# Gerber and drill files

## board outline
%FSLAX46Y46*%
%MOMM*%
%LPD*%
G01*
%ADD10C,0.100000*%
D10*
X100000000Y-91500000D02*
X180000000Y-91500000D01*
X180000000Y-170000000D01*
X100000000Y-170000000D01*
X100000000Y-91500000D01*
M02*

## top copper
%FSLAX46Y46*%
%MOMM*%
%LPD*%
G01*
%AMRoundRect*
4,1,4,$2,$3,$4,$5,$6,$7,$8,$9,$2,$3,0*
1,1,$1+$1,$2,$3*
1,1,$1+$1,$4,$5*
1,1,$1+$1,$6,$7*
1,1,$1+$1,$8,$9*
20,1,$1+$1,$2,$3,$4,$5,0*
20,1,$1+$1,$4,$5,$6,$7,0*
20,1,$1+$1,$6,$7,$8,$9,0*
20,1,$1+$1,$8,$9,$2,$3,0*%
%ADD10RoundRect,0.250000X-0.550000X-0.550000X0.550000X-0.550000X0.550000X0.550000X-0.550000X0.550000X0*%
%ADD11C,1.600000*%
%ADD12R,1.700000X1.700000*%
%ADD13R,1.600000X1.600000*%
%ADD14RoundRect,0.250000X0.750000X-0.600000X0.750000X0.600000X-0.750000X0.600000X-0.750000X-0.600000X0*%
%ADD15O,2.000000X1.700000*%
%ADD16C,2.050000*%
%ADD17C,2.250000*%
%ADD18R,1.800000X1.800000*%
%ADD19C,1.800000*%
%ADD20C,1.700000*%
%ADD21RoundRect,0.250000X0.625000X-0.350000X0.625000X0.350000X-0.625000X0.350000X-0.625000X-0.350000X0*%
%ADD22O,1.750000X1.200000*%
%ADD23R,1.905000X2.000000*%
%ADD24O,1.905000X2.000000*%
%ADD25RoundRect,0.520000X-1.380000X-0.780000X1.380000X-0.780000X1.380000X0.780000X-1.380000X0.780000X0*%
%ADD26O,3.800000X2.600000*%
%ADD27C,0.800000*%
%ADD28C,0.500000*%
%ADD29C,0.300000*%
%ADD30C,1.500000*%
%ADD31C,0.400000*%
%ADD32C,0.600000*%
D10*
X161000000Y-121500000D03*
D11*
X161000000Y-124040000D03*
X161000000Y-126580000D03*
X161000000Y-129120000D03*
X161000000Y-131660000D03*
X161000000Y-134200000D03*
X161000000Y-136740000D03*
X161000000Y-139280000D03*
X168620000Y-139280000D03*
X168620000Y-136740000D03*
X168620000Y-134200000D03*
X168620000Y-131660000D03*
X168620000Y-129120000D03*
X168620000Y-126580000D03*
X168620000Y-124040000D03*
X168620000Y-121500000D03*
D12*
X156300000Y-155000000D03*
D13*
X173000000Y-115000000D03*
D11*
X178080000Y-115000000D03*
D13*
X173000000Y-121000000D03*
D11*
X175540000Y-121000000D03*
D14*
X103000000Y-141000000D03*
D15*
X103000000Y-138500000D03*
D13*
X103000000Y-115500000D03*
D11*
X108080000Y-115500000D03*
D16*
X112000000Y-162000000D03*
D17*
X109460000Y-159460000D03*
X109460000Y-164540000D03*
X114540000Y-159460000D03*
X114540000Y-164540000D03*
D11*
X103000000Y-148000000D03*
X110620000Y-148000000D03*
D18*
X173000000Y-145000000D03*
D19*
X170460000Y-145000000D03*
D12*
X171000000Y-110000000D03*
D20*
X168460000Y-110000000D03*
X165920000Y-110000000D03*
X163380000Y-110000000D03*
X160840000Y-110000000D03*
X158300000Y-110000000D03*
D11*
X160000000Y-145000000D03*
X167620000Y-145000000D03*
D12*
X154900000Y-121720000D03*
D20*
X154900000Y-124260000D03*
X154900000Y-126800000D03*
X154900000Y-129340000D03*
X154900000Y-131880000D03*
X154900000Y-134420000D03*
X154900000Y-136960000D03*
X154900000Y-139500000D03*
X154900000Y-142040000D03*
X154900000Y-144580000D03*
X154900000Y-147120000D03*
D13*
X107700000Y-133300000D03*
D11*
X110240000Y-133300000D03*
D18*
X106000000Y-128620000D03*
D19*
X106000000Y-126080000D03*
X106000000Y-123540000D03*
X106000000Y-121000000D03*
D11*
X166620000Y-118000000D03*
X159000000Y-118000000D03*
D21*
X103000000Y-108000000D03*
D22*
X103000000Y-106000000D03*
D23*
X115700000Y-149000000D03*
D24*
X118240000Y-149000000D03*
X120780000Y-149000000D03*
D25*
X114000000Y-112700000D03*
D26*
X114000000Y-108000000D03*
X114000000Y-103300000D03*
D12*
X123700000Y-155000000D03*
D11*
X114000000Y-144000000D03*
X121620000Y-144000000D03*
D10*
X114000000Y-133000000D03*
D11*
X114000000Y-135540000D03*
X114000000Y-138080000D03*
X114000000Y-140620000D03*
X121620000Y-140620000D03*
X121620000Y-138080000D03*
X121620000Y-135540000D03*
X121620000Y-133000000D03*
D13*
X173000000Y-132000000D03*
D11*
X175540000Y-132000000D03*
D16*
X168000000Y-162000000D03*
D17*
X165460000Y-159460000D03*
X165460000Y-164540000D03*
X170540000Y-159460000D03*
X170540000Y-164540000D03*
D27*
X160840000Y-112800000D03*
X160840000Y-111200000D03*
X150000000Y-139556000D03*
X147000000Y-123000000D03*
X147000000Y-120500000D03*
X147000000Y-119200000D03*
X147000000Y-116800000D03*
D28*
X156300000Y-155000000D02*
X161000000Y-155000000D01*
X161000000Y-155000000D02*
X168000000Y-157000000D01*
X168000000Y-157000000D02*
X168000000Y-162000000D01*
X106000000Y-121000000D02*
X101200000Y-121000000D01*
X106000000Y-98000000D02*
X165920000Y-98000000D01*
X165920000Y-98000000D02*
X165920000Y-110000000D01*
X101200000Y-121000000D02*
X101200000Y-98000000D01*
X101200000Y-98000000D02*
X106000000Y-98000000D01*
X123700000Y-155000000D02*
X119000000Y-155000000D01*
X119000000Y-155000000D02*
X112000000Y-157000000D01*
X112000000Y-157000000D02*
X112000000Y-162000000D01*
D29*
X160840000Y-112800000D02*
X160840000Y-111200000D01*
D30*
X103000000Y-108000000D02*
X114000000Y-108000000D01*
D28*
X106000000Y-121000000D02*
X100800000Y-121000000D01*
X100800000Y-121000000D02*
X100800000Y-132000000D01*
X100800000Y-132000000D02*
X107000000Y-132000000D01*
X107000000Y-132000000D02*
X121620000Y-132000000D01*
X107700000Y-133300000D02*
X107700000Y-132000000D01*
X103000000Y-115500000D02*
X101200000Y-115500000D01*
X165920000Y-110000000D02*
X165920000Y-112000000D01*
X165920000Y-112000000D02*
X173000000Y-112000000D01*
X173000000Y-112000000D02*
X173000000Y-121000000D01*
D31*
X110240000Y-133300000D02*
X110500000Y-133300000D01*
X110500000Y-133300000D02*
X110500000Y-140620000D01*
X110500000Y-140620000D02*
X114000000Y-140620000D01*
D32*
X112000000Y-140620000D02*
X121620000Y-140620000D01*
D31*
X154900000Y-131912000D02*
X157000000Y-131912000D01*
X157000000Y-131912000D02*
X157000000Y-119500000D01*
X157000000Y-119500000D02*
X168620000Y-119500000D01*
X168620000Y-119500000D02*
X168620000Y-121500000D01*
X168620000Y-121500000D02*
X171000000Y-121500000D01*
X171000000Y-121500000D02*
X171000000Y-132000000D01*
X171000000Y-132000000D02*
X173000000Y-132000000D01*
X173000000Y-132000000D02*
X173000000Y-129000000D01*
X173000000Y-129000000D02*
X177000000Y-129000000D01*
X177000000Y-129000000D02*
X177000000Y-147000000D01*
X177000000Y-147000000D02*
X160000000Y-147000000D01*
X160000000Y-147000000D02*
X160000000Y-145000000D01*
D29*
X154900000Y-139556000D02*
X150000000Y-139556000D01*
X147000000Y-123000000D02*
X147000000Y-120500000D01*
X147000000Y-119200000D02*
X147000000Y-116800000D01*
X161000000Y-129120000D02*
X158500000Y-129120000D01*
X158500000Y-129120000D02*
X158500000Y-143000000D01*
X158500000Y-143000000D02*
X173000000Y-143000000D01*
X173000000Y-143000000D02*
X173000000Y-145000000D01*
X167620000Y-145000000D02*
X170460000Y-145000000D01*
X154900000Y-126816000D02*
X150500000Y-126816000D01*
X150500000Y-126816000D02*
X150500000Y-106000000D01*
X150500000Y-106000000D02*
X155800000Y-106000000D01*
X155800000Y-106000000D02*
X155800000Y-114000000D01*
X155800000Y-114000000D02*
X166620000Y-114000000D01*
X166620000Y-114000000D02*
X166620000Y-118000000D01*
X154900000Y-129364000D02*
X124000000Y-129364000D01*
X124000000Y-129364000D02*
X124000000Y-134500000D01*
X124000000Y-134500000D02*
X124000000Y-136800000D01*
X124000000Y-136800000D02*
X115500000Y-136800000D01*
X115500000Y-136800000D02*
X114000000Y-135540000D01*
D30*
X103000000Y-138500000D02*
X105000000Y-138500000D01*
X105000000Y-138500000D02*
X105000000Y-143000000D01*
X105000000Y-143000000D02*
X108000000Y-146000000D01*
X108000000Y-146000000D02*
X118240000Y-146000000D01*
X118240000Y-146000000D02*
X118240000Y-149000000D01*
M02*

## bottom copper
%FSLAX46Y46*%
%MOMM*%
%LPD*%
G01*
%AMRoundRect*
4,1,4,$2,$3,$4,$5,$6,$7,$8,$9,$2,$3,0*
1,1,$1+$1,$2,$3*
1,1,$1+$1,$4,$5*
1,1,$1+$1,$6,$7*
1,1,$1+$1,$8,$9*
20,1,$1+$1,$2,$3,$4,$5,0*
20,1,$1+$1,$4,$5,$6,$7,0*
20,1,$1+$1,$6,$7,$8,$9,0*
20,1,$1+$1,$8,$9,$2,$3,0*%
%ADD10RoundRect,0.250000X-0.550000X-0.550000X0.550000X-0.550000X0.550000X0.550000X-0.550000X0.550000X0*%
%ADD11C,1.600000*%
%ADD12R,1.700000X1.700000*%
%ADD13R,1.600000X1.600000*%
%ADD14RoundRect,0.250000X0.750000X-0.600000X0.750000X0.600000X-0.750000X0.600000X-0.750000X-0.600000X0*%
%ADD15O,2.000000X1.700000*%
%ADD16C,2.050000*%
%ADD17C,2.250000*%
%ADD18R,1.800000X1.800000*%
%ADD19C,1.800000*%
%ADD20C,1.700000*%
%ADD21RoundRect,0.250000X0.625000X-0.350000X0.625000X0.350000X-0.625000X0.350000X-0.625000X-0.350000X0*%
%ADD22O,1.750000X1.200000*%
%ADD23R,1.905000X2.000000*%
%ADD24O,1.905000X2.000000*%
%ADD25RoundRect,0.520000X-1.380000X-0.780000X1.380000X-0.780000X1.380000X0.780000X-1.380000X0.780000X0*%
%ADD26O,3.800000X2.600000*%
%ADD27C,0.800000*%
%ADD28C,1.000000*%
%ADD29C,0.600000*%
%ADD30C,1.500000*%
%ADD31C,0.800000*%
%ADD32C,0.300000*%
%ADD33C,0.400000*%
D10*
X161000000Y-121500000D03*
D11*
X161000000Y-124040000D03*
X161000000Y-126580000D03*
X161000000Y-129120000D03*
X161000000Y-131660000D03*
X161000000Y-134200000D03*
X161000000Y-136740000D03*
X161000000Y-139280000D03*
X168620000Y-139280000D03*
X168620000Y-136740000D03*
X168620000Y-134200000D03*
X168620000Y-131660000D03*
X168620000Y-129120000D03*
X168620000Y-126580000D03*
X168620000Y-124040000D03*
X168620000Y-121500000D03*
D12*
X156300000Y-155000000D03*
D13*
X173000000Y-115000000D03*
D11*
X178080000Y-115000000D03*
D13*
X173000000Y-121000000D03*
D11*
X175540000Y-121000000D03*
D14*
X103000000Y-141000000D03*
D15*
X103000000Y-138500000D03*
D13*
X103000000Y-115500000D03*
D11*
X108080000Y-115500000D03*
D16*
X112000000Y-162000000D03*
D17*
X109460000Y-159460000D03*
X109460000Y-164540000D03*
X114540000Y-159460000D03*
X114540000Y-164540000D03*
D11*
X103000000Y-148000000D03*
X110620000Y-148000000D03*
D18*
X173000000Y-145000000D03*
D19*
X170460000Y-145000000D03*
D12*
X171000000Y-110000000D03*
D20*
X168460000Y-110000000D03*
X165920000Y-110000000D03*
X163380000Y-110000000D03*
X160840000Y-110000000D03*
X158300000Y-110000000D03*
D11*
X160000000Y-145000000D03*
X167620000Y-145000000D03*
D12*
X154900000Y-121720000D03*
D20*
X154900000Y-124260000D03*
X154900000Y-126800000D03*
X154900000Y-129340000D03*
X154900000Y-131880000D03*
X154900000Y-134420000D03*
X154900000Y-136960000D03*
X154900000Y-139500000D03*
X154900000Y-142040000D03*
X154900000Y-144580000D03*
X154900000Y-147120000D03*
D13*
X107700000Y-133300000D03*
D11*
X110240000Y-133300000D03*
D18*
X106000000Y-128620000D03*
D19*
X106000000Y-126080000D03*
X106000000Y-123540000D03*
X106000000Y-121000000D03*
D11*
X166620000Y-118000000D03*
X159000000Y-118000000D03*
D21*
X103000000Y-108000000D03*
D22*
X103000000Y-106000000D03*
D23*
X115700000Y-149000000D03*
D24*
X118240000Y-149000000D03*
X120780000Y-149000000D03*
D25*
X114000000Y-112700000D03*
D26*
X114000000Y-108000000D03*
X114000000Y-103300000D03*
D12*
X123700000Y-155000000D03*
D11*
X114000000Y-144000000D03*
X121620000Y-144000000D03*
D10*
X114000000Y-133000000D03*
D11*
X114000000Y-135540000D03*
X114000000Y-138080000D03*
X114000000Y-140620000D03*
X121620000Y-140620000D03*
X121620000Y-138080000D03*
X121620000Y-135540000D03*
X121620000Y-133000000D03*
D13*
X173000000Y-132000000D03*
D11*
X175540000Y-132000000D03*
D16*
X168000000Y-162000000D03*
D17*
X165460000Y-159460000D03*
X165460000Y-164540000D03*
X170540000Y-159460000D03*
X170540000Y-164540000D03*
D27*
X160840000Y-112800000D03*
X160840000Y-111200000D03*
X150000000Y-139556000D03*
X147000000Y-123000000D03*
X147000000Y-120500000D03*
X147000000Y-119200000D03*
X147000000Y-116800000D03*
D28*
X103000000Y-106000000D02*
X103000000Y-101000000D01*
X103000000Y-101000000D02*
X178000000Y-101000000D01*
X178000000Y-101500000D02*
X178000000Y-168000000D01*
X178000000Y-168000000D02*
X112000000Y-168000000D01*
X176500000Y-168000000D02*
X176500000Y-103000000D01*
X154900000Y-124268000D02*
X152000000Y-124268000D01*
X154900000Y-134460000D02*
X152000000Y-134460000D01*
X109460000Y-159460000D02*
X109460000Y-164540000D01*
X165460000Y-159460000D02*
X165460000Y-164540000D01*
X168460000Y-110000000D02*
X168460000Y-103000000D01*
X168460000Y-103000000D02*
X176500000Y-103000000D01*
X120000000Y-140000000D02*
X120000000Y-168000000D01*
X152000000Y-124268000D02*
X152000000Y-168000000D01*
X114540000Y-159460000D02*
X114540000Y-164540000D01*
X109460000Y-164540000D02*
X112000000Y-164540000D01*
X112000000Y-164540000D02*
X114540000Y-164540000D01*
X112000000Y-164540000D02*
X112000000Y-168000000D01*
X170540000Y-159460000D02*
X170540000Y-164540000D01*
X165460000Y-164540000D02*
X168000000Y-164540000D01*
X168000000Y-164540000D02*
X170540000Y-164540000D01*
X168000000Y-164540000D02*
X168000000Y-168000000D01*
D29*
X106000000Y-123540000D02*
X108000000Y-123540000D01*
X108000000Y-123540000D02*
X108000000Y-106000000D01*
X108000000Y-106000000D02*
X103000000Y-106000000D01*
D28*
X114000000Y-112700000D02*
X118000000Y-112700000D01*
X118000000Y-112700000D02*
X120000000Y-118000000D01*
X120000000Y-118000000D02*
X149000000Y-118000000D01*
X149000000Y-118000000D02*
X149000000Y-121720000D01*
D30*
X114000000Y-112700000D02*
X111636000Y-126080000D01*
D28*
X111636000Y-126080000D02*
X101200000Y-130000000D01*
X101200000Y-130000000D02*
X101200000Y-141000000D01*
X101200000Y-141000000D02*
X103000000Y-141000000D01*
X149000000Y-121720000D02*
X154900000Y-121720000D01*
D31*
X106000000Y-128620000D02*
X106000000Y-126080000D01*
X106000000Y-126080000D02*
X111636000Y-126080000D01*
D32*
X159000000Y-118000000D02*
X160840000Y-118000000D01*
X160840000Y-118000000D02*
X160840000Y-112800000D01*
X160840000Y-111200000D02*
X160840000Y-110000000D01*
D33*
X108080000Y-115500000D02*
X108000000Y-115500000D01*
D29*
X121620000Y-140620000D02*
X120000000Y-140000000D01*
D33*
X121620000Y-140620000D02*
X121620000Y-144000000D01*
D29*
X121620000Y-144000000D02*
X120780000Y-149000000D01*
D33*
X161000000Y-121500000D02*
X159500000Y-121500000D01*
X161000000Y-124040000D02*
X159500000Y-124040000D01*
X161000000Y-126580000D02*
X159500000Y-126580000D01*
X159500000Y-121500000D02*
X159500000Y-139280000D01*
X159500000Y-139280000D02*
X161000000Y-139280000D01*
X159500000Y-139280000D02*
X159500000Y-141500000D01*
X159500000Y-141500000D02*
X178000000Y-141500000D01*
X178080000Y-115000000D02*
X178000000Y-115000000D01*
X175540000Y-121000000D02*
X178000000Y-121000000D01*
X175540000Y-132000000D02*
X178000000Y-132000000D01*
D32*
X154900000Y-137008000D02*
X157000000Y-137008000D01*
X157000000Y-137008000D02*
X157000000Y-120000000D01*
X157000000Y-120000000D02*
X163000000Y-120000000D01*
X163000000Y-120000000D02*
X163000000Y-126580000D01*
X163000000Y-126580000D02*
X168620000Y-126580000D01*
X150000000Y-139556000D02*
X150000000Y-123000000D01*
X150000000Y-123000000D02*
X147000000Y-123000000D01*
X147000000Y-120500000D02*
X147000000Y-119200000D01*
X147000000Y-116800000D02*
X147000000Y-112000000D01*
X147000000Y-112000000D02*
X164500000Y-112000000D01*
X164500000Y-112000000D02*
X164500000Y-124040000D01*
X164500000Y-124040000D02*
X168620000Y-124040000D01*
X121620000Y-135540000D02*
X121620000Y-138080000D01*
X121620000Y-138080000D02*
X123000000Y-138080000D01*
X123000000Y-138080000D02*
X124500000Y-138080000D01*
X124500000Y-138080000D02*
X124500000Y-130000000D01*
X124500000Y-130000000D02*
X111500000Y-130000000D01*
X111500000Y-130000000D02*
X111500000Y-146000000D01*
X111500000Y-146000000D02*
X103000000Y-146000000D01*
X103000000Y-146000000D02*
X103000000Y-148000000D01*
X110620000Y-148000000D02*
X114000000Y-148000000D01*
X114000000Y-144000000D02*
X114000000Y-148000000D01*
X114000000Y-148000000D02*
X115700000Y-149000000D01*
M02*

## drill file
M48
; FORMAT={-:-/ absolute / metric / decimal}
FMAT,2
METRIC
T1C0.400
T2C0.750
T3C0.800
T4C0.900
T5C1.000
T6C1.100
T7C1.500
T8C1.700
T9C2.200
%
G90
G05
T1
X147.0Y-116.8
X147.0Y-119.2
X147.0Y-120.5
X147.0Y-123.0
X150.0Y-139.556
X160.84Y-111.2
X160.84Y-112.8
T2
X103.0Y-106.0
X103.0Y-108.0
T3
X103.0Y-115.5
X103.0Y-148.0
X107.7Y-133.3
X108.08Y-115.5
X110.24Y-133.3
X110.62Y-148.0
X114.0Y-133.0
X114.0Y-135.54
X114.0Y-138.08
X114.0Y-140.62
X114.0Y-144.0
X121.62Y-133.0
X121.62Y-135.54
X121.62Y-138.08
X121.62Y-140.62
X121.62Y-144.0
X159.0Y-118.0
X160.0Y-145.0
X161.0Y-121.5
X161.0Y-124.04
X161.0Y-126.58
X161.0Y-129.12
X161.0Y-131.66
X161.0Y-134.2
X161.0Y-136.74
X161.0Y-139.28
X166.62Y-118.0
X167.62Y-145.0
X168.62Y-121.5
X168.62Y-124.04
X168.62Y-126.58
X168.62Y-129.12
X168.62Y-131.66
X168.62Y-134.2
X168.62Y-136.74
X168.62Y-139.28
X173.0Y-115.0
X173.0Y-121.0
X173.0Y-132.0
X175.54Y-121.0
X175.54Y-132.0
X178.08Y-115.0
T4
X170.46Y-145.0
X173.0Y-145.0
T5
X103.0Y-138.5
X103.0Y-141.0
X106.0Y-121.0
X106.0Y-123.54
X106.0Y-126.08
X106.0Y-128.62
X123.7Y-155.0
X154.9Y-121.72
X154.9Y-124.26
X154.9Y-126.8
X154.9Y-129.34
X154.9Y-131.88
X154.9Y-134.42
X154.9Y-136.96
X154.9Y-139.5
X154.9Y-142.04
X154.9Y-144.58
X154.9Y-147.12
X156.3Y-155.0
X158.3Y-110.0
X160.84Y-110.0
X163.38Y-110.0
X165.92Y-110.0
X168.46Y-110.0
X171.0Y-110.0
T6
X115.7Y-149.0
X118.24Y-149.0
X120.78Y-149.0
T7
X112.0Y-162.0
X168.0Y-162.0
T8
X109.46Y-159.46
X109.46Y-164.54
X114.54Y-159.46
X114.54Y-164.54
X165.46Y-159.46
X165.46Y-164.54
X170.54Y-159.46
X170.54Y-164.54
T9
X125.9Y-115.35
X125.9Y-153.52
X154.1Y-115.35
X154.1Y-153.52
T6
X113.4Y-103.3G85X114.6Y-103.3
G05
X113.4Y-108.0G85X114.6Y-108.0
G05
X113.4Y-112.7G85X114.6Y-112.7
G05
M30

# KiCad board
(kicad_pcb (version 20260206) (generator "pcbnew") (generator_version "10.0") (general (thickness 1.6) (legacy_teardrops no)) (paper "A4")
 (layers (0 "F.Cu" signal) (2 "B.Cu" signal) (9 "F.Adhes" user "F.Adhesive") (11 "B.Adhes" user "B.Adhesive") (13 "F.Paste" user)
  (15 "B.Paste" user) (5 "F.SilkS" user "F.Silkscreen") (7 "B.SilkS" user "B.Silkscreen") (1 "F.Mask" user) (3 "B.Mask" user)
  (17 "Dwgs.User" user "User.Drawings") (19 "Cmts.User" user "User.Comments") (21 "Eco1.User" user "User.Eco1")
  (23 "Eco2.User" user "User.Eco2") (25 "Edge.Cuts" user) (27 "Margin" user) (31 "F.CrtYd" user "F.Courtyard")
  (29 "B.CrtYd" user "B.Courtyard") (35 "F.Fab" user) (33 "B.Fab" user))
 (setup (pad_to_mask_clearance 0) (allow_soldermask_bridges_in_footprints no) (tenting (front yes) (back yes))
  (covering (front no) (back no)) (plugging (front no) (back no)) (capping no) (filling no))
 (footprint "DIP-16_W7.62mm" (layer "F.Cu") (at 161 121.5)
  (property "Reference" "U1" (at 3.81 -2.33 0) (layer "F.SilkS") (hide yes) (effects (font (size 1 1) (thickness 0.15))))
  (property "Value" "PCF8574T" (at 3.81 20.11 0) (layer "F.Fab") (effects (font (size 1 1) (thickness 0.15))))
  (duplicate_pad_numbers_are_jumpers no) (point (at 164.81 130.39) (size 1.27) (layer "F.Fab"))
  (pad "1" thru_hole roundrect (at 0 0) (size 1.6 1.6) (drill 0.8) (layers "*.Cu" "*.Mask") (remove_unused_layers no)
   (roundrect_rratio 0.15625) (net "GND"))
  (pad "2" thru_hole circle (at 0 2.54) (size 1.6 1.6) (drill 0.8) (layers "*.Cu" "*.Mask") (remove_unused_layers no) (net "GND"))
  (pad "3" thru_hole circle (at 0 5.08) (size 1.6 1.6) (drill 0.8) (layers "*.Cu" "*.Mask") (remove_unused_layers no) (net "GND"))
  (pad "4" thru_hole circle (at 0 7.62) (size 1.6 1.6) (drill 0.8) (layers "*.Cu" "*.Mask") (remove_unused_layers no) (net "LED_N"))
  (pad "5" thru_hole circle (at 0 10.16) (size 1.6 1.6) (drill 0.8) (layers "*.Cu" "*.Mask") (remove_unused_layers no))
  (pad "6" thru_hole circle (at 0 12.7) (size 1.6 1.6) (drill 0.8) (layers "*.Cu" "*.Mask") (remove_unused_layers no))
  (pad "7" thru_hole circle (at 0 15.24) (size 1.6 1.6) (drill 0.8) (layers "*.Cu" "*.Mask") (remove_unused_layers no))
  (pad "8" thru_hole circle (at 0 17.78) (size 1.6 1.6) (drill 0.8) (layers "*.Cu" "*.Mask") (remove_unused_layers no) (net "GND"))
  (pad "9" thru_hole circle (at 7.62 17.78) (size 1.6 1.6) (drill 0.8) (layers "*.Cu" "*.Mask") (remove_unused_layers no))
  (pad "10" thru_hole circle (at 7.62 15.24) (size 1.6 1.6) (drill 0.8) (layers "*.Cu" "*.Mask") (remove_unused_layers no))
  (pad "11" thru_hole circle (at 7.62 12.7) (size 1.6 1.6) (drill 0.8) (layers "*.Cu" "*.Mask") (remove_unused_layers no))
  (pad "12" thru_hole circle (at 7.62 10.16) (size 1.6 1.6) (drill 0.8) (layers "*.Cu" "*.Mask") (remove_unused_layers no))
  (pad "13" thru_hole circle (at 7.62 7.62) (size 1.6 1.6) (drill 0.8) (layers "*.Cu" "*.Mask") (remove_unused_layers no))
  (pad "14" thru_hole circle (at 7.62 5.08) (size 1.6 1.6) (drill 0.8) (layers "*.Cu" "*.Mask") (remove_unused_layers no) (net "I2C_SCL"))
  (pad "15" thru_hole circle (at 7.62 2.54) (size 1.6 1.6) (drill 0.8) (layers "*.Cu" "*.Mask") (remove_unused_layers no) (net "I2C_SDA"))
  (pad "16" thru_hole circle (at 7.62 0) (size 1.6 1.6) (drill 0.8) (layers "*.Cu" "*.Mask") (remove_unused_layers no) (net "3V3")))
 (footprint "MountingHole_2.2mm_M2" (layer "F.Cu") (at 154.1 115.35)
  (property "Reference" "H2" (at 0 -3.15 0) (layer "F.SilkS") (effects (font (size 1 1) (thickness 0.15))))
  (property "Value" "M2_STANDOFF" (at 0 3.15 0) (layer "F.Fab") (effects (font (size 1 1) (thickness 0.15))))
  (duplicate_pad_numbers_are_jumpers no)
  (pad "" np_thru_hole circle (at 0 0) (size 2.2 2.2) (drill 2.2) (layers "*.Cu" "*.Mask")))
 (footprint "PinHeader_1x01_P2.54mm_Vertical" (layer "F.Cu") (at 156.3 155)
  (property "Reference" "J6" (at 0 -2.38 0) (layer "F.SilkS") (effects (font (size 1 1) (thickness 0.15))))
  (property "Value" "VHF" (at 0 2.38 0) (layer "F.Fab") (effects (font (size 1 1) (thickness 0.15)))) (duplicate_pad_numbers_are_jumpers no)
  (pad "1" thru_hole rect (at 0 0) (size 1.7 1.7) (drill 1) (layers "*.Cu" "*.Mask") (remove_unused_layers no) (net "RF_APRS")))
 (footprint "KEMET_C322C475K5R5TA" (layer "F.Cu") (at 173 115)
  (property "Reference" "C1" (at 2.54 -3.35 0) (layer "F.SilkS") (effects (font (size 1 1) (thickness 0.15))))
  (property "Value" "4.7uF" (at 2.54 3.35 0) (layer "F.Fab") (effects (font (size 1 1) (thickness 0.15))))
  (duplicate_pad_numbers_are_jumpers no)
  (pad "1" thru_hole rect (at 0 0) (size 1.6 1.6) (drill 0.8) (layers "*.Cu" "*.Mask") (remove_unused_layers no) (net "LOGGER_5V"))
  (pad "2" thru_hole circle (at 5.08 0) (size 1.6 1.6) (drill 0.8) (layers "*.Cu" "*.Mask") (remove_unused_layers no) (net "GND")))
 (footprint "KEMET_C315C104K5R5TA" (layer "F.Cu") (at 173 121)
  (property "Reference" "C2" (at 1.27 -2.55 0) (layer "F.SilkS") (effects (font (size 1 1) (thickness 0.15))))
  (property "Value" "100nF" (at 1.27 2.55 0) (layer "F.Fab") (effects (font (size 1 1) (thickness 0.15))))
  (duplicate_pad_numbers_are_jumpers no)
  (pad "1" thru_hole rect (at 0 0) (size 1.6 1.6) (drill 0.8) (layers "*.Cu" "*.Mask") (remove_unused_layers no) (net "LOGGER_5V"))
  (pad "2" thru_hole circle (at 2.54 0) (size 1.6 1.6) (drill 0.8) (layers "*.Cu" "*.Mask") (remove_unused_layers no) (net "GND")))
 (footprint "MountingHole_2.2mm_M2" (layer "F.Cu") (at 125.9 153.52)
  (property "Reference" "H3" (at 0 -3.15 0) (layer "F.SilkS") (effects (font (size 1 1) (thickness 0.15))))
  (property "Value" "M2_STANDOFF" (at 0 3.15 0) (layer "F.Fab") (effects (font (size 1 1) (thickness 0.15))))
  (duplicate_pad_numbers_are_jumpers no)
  (pad "" np_thru_hole circle (at 0 0) (size 2.2 2.2) (drill 2.2) (layers "*.Cu" "*.Mask")))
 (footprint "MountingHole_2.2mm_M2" (layer "F.Cu") (at 154.1 153.52)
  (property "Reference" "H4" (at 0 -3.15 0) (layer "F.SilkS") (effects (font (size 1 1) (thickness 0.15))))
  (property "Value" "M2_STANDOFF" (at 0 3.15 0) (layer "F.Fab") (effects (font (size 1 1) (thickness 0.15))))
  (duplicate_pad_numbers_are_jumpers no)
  (pad "" np_thru_hole circle (at 0 0) (size 2.2 2.2) (drill 2.2) (layers "*.Cu" "*.Mask")))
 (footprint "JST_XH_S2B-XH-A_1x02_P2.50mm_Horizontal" (layer "F.Cu") (at 103 141 90)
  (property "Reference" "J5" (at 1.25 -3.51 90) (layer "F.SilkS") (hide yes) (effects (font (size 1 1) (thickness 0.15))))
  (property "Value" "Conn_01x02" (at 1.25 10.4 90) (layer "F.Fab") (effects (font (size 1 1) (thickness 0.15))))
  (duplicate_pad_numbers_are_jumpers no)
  (pad "1" thru_hole roundrect (at 0 0 90) (size 1.7 2) (drill 1) (layers "*.Cu" "*.Mask") (remove_unused_layers no)
   (roundrect_rratio 0.147059) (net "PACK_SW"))
  (pad "2" thru_hole oval (at 2.5 0 90) (size 1.7 2) (drill 1) (layers "*.Cu" "*.Mask") (remove_unused_layers no) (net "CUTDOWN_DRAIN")))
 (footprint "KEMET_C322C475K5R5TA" (layer "F.Cu") (at 103 115.5)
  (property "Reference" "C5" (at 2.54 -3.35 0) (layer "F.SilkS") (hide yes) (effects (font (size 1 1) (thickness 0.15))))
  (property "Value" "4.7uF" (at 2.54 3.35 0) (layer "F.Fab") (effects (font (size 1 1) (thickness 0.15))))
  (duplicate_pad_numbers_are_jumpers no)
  (pad "1" thru_hole rect (at 0 0) (size 1.6 1.6) (drill 0.8) (layers "*.Cu" "*.Mask") (remove_unused_layers no) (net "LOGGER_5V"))
  (pad "2" thru_hole circle (at 5.08 0) (size 1.6 1.6) (drill 0.8) (layers "*.Cu" "*.Mask") (remove_unused_layers no) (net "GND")))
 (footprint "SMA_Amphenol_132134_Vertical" (layer "F.Cu") (at 112 162)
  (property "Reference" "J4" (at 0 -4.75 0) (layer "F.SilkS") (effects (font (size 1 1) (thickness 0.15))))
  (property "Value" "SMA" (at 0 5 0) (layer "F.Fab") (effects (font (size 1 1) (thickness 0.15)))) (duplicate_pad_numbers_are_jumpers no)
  (pad "1" thru_hole circle (at 0 0) (size 2.05 2.05) (drill 1.5) (layers "*.Cu" "*.Mask") (remove_unused_layers no) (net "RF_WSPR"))
  (pad "2" thru_hole circle (at -2.54 -2.54) (size 2.25 2.25) (drill 1.7) (layers "*.Cu" "*.Mask") (remove_unused_layers no) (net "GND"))
  (pad "2" thru_hole circle (at -2.54 2.54) (size 2.25 2.25) (drill 1.7) (layers "*.Cu" "*.Mask") (remove_unused_layers no) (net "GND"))
  (pad "2" thru_hole circle (at 2.54 -2.54) (size 2.25 2.25) (drill 1.7) (layers "*.Cu" "*.Mask") (remove_unused_layers no) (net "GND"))
  (pad "2" thru_hole circle (at 2.54 2.54) (size 2.25 2.25) (drill 1.7) (layers "*.Cu" "*.Mask") (remove_unused_layers no) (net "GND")))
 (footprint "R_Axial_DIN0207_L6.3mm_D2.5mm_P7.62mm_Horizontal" (layer "F.Cu") (at 103 148)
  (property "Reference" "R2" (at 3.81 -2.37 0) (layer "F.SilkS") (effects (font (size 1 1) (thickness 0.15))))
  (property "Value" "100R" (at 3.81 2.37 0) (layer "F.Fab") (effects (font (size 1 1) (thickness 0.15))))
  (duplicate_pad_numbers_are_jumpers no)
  (pad "1" thru_hole circle (at 0 0) (size 1.6 1.6) (drill 0.8) (layers "*.Cu" "*.Mask") (remove_unused_layers no) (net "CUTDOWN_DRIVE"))
  (pad "2" thru_hole circle (at 7.62 0) (size 1.6 1.6) (drill 0.8) (layers "*.Cu" "*.Mask") (remove_unused_layers no) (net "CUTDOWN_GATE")))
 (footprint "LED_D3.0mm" (layer "F.Cu") (at 173 145 180)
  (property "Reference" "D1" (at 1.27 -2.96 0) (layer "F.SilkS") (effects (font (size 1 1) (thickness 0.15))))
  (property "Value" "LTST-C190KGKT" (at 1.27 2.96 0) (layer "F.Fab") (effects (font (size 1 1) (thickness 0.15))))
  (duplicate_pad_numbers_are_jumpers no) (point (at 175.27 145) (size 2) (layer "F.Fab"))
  (pad "1" thru_hole rect (at 0 0) (size 1.8 1.8) (drill 0.9) (layers "*.Cu" "*.Mask") (remove_unused_layers no) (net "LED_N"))
  (pad "2" thru_hole circle (at 2.54 0) (size 1.8 1.8) (drill 0.9) (layers "*.Cu" "*.Mask") (remove_unused_layers no) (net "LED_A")))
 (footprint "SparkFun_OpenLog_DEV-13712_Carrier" (layer "F.Cu") (at 171 110)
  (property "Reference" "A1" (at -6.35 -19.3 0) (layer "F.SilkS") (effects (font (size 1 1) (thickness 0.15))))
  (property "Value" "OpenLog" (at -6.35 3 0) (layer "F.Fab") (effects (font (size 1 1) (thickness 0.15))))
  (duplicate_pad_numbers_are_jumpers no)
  (pad "1" thru_hole rect (at 0 0) (size 1.7 1.7) (drill 1) (layers "*.Cu" "*.Mask") (remove_unused_layers no))
  (pad "2" thru_hole circle (at -2.54 0) (size 1.7 1.7) (drill 1) (layers "*.Cu" "*.Mask") (remove_unused_layers no) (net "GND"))
  (pad "3" thru_hole circle (at -5.08 0) (size 1.7 1.7) (drill 1) (layers "*.Cu" "*.Mask") (remove_unused_layers no) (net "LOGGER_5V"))
  (pad "4" thru_hole circle (at -7.62 0) (size 1.7 1.7) (drill 1) (layers "*.Cu" "*.Mask") (remove_unused_layers no))
  (pad "5" thru_hole circle (at -10.16 0) (size 1.7 1.7) (drill 1) (layers "*.Cu" "*.Mask") (remove_unused_layers no) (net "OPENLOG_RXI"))
  (pad "6" thru_hole circle (at -12.7 0) (size 1.7 1.7) (drill 1) (layers "*.Cu" "*.Mask") (remove_unused_layers no)))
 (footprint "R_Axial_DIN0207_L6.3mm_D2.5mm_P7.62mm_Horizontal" (layer "F.Cu") (at 160 145)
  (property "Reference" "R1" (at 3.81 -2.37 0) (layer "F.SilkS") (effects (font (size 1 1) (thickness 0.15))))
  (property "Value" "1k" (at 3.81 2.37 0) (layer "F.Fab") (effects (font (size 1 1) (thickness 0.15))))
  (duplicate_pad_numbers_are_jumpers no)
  (pad "1" thru_hole circle (at 0 0) (size 1.6 1.6) (drill 0.8) (layers "*.Cu" "*.Mask") (remove_unused_layers no) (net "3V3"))
  (pad "2" thru_hole circle (at 7.62 0) (size 1.6 1.6) (drill 0.8) (layers "*.Cu" "*.Mask") (remove_unused_layers no) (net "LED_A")))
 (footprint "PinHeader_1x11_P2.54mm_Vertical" (layer "F.Cu") (at 154.9 121.72)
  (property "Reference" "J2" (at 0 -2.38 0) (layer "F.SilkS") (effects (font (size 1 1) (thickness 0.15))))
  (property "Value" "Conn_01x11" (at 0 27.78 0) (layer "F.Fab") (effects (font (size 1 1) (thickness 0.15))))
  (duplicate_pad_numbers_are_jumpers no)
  (pad "1" thru_hole rect (at 0 0) (size 1.7 1.7) (drill 1) (layers "*.Cu" "*.Mask") (remove_unused_layers no) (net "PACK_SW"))
  (pad "2" thru_hole circle (at 0 2.54) (size 1.7 1.7) (drill 1) (layers "*.Cu" "*.Mask") (remove_unused_layers no) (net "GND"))
  (pad "3" thru_hole circle (at 0 5.08) (size 1.7 1.7) (drill 1) (layers "*.Cu" "*.Mask") (remove_unused_layers no) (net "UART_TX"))
  (pad "4" thru_hole circle (at 0 7.62) (size 1.7 1.7) (drill 1) (layers "*.Cu" "*.Mask") (remove_unused_layers no) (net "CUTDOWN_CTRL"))
  (pad "5" thru_hole circle (at 0 10.16) (size 1.7 1.7) (drill 1) (layers "*.Cu" "*.Mask") (remove_unused_layers no) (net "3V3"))
  (pad "6" thru_hole circle (at 0 12.7) (size 1.7 1.7) (drill 1) (layers "*.Cu" "*.Mask") (remove_unused_layers no) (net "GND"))
  (pad "7" thru_hole circle (at 0 15.24) (size 1.7 1.7) (drill 1) (layers "*.Cu" "*.Mask") (remove_unused_layers no) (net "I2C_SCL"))
  (pad "8" thru_hole circle (at 0 17.78) (size 1.7 1.7) (drill 1) (layers "*.Cu" "*.Mask") (remove_unused_layers no) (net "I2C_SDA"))
  (pad "9" thru_hole circle (at 0 20.32) (size 1.7 1.7) (drill 1) (layers "*.Cu" "*.Mask") (remove_unused_layers no))
  (pad "10" thru_hole circle (at 0 22.86) (size 1.7 1.7) (drill 1) (layers "*.Cu" "*.Mask") (remove_unused_layers no))
  (pad "11" thru_hole circle (at 0 25.4) (size 1.7 1.7) (drill 1) (layers "*.Cu" "*.Mask") (remove_unused_layers no)))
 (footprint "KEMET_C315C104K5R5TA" (layer "F.Cu") (at 107.7 133.3)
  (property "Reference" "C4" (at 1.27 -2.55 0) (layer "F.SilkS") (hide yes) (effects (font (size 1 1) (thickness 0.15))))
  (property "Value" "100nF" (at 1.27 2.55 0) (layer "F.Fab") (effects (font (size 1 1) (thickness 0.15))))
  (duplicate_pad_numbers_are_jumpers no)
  (pad "1" thru_hole rect (at 0 0) (size 1.6 1.6) (drill 0.8) (layers "*.Cu" "*.Mask") (remove_unused_layers no) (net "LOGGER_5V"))
  (pad "2" thru_hole circle (at 2.54 0) (size 1.6 1.6) (drill 0.8) (layers "*.Cu" "*.Mask") (remove_unused_layers no) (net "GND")))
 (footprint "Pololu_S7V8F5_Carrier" (layer "F.Cu") (at 106 121 -90)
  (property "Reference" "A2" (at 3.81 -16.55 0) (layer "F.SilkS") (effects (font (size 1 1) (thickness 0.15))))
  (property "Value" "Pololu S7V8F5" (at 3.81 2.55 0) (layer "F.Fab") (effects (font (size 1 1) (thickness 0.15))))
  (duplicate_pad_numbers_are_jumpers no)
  (pad "1" thru_hole rect (at 7.62 0) (size 1.8 1.8) (drill 1) (layers "*.Cu" "*.Mask") (remove_unused_layers no) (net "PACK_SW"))
  (pad "2" thru_hole circle (at 5.08 0) (size 1.8 1.8) (drill 1) (layers "*.Cu" "*.Mask") (remove_unused_layers no) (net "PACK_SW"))
  (pad "3" thru_hole circle (at 2.54 0) (size 1.8 1.8) (drill 1) (layers "*.Cu" "*.Mask") (remove_unused_layers no) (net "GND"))
  (pad "4" thru_hole circle (at 0 0) (size 1.8 1.8) (drill 1) (layers "*.Cu" "*.Mask") (remove_unused_layers no) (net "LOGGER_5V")))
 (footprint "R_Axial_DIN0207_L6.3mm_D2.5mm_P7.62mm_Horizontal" (layer "F.Cu") (at 166.62 118 180)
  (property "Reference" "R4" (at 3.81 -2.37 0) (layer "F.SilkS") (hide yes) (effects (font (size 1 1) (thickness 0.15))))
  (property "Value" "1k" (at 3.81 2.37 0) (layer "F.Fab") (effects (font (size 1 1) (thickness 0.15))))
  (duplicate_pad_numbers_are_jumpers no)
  (pad "1" thru_hole circle (at 0 0 180) (size 1.6 1.6) (drill 0.8) (layers "*.Cu" "*.Mask") (remove_unused_layers no) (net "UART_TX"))
  (pad "2" thru_hole circle (at 7.62 0 180) (size 1.6 1.6) (drill 0.8) (layers "*.Cu" "*.Mask") (remove_unused_layers no)
   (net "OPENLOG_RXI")))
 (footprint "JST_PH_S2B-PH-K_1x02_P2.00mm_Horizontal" (layer "F.Cu") (at 103 108 90)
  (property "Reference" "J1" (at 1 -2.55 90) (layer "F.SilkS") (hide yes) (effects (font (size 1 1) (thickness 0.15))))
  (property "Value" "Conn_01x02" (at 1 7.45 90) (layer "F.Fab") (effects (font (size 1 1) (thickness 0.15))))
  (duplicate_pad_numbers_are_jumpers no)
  (pad "1" thru_hole roundrect (at 0 0 90) (size 1.2 1.75) (drill 0.75) (layers "*.Cu" "*.Mask") (remove_unused_layers no)
   (roundrect_rratio 0.208333) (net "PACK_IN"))
  (pad "2" thru_hole oval (at 2 0 90) (size 1.2 1.75) (drill 0.75) (layers "*.Cu" "*.Mask") (remove_unused_layers no) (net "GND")))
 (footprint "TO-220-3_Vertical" (layer "F.Cu") (at 115.7 149)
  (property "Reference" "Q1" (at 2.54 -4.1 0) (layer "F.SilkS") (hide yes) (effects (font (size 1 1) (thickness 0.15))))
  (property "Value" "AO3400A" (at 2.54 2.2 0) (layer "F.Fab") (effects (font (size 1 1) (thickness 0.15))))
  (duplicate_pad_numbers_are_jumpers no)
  (pad "1" thru_hole rect (at 0 0) (size 1.905 2) (drill 1.1) (layers "*.Cu" "*.Mask") (remove_unused_layers no) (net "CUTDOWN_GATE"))
  (pad "2" thru_hole oval (at 2.54 0) (size 1.905 2) (drill 1.1) (layers "*.Cu" "*.Mask") (remove_unused_layers no) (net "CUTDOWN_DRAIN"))
  (pad "3" thru_hole oval (at 5.08 0) (size 1.905 2) (drill 1.1) (layers "*.Cu" "*.Mask") (remove_unused_layers no) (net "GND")))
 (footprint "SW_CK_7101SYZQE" (layer "F.Cu") (at 114 108)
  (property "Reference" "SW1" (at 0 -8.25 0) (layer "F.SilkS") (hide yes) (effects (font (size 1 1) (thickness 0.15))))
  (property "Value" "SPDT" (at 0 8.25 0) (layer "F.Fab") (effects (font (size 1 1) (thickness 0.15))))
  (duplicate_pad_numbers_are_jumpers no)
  (pad "1" thru_hole roundrect (at 0 4.7) (size 3.8 2.6) (drill oval 2.3 1.1) (layers "*.Cu" "*.Mask") (remove_unused_layers no)
   (roundrect_rratio 0.2) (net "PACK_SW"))
  (pad "2" thru_hole oval (at 0 0) (size 3.8 2.6) (drill oval 2.3 1.1) (layers "*.Cu" "*.Mask") (remove_unused_layers no) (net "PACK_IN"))
  (pad "3" thru_hole oval (at 0 -4.7) (size 3.8 2.6) (drill oval 2.3 1.1) (layers "*.Cu" "*.Mask") (remove_unused_layers no)))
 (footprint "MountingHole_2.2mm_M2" (layer "F.Cu") (at 125.9 115.35)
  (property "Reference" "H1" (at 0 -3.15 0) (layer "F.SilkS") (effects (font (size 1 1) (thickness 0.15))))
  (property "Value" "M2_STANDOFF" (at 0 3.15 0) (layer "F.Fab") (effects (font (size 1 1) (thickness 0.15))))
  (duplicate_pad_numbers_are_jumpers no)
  (pad "" np_thru_hole circle (at 0 0) (size 2.2 2.2) (drill 2.2) (layers "*.Cu" "*.Mask")))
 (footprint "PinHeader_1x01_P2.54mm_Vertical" (layer "F.Cu") (at 123.7 155)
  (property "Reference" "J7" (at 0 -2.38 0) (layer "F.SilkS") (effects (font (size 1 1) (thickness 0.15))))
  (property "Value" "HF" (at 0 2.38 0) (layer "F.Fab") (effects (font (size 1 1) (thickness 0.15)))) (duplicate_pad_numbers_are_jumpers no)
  (pad "1" thru_hole rect (at 0 0) (size 1.7 1.7) (drill 1) (layers "*.Cu" "*.Mask") (remove_unused_layers no) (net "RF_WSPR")))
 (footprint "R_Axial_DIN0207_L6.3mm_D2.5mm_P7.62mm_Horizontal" (layer "F.Cu") (at 114 144)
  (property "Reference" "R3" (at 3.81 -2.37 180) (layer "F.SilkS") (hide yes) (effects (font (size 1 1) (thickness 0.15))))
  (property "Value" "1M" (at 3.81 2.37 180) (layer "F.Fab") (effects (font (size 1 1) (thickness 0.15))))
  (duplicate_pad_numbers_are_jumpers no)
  (pad "1" thru_hole circle (at 0 0 180) (size 1.6 1.6) (drill 0.8) (layers "*.Cu" "*.Mask") (remove_unused_layers no) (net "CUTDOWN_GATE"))
  (pad "2" thru_hole circle (at 7.62 0 180) (size 1.6 1.6) (drill 0.8) (layers "*.Cu" "*.Mask") (remove_unused_layers no) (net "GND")))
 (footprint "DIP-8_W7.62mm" (layer "F.Cu") (at 114 133)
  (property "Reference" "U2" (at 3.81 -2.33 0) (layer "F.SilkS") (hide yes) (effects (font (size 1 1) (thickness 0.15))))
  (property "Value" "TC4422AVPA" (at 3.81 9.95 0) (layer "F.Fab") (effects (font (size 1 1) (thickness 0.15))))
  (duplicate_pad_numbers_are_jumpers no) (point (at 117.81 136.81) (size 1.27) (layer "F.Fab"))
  (pad "1" thru_hole roundrect (at 0 0) (size 1.6 1.6) (drill 0.8) (layers "*.Cu" "*.Mask") (remove_unused_layers no)
   (roundrect_rratio 0.15625) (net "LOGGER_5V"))
  (pad "2" thru_hole circle (at 0 2.54) (size 1.6 1.6) (drill 0.8) (layers "*.Cu" "*.Mask") (remove_unused_layers no) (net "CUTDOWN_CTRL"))
  (pad "3" thru_hole circle (at 0 5.08) (size 1.6 1.6) (drill 0.8) (layers "*.Cu" "*.Mask") (remove_unused_layers no))
  (pad "4" thru_hole circle (at 0 7.62) (size 1.6 1.6) (drill 0.8) (layers "*.Cu" "*.Mask") (remove_unused_layers no) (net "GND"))
  (pad "5" thru_hole circle (at 7.62 7.62) (size 1.6 1.6) (drill 0.8) (layers "*.Cu" "*.Mask") (remove_unused_layers no) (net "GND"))
  (pad "6" thru_hole circle (at 7.62 5.08) (size 1.6 1.6) (drill 0.8) (layers "*.Cu" "*.Mask") (remove_unused_layers no)
   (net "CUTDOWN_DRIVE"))
  (pad "7" thru_hole circle (at 7.62 2.54) (size 1.6 1.6) (drill 0.8) (layers "*.Cu" "*.Mask") (remove_unused_layers no)
   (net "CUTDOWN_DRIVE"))
  (pad "8" thru_hole circle (at 7.62 0) (size 1.6 1.6) (drill 0.8) (layers "*.Cu" "*.Mask") (remove_unused_layers no) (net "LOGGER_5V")))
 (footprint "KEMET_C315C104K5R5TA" (layer "F.Cu") (at 173 132)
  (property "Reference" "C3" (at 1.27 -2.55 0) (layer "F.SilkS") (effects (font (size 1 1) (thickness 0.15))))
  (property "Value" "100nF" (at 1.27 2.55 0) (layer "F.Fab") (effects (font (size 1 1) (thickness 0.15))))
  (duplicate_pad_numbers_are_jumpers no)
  (pad "1" thru_hole rect (at 0 0) (size 1.6 1.6) (drill 0.8) (layers "*.Cu" "*.Mask") (remove_unused_layers no) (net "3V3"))
  (pad "2" thru_hole circle (at 2.54 0) (size 1.6 1.6) (drill 0.8) (layers "*.Cu" "*.Mask") (remove_unused_layers no) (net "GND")))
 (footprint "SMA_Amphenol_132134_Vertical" (layer "F.Cu") (at 168 162)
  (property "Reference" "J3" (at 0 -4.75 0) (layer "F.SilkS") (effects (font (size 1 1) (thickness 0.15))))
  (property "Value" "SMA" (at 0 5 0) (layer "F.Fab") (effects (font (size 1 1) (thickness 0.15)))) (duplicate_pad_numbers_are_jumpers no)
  (pad "1" thru_hole circle (at 0 0) (size 2.05 2.05) (drill 1.5) (layers "*.Cu" "*.Mask") (remove_unused_layers no) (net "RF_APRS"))
  (pad "2" thru_hole circle (at -2.54 -2.54) (size 2.25 2.25) (drill 1.7) (layers "*.Cu" "*.Mask") (remove_unused_layers no) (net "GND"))
  (pad "2" thru_hole circle (at -2.54 2.54) (size 2.25 2.25) (drill 1.7) (layers "*.Cu" "*.Mask") (remove_unused_layers no) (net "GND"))
  (pad "2" thru_hole circle (at 2.54 -2.54) (size 2.25 2.25) (drill 1.7) (layers "*.Cu" "*.Mask") (remove_unused_layers no) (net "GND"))
  (pad "2" thru_hole circle (at 2.54 2.54) (size 2.25 2.25) (drill 1.7) (layers "*.Cu" "*.Mask") (remove_unused_layers no) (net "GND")))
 (gr_rect (start 100 91.5) (end 180 170) (stroke (width 0.1) (type default)) (fill no) (layer "Edge.Cuts"))
 (segment (start 103 106) (end 103 101) (width 1) (layer "B.Cu") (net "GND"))
 (segment (start 103 101) (end 178 101) (width 1) (layer "B.Cu") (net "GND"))
 (segment (start 178 101.5) (end 178 168) (width 1) (layer "B.Cu") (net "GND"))
 (segment (start 178 168) (end 112 168) (width 1) (layer "B.Cu") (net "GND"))
 (segment (start 176.5 168) (end 176.5 103) (width 1) (layer "B.Cu") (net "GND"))
 (segment (start 154.9 124.268) (end 152 124.268) (width 1) (layer "B.Cu") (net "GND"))
 (segment (start 154.9 134.46) (end 152 134.46) (width 1) (layer "B.Cu") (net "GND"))
 (segment (start 109.46 159.46) (end 109.46 164.54) (width 1) (layer "B.Cu") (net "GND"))
 (segment (start 165.46 159.46) (end 165.46 164.54) (width 1) (layer "B.Cu") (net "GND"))
 (segment (start 168.46 110) (end 168.46 103) (width 1) (layer "B.Cu") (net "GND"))
 (segment (start 168.46 103) (end 176.5 103) (width 1) (layer "B.Cu") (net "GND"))
 (segment (start 120 140) (end 120 168) (width 1) (layer "B.Cu") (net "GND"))
 (segment (start 152 124.268) (end 152 168) (width 1) (layer "B.Cu") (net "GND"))
 (segment (start 114.54 159.46) (end 114.54 164.54) (width 1) (layer "B.Cu") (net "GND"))
 (segment (start 109.46 164.54) (end 112 164.54) (width 1) (layer "B.Cu") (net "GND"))
 (segment (start 112 164.54) (end 114.54 164.54) (width 1) (layer "B.Cu") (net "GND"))
 (segment (start 112 164.54) (end 112 168) (width 1) (layer "B.Cu") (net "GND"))
 (segment (start 170.54 159.46) (end 170.54 164.54) (width 1) (layer "B.Cu") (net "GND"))
 (segment (start 165.46 164.54) (end 168 164.54) (width 1) (layer "B.Cu") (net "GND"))
 (segment (start 168 164.54) (end 170.54 164.54) (width 1) (layer "B.Cu") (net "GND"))
 (segment (start 168 164.54) (end 168 168) (width 1) (layer "B.Cu") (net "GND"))
 (segment (start 106 123.54) (end 108 123.54) (width 0.6) (layer "B.Cu") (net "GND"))
 (segment (start 108 123.54) (end 108 106) (width 0.6) (layer "B.Cu") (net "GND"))
 (segment (start 108 106) (end 103 106) (width 0.6) (layer "B.Cu") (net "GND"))
 (segment (start 156.3 155) (end 161 155) (width 0.5) (layer "F.Cu") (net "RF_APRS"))
 (segment (start 161 155) (end 168 157) (width 0.5) (layer "F.Cu") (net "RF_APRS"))
 (segment (start 168 157) (end 168 162) (width 0.5) (layer "F.Cu") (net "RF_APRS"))
 (segment (start 106 121) (end 101.2 121) (width 0.5) (layer "F.Cu") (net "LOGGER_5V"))
 (segment (start 106 98) (end 165.92 98) (width 0.5) (layer "F.Cu") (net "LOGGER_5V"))
 (segment (start 165.92 98) (end 165.92 110) (width 0.5) (layer "F.Cu") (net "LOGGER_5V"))
 (segment (start 101.2 121) (end 101.2 98) (width 0.5) (layer "F.Cu") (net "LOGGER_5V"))
 (segment (start 101.2 98) (end 106 98) (width 0.5) (layer "F.Cu") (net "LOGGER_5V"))
 (segment (start 114 112.7) (end 118 112.7) (width 1) (layer "B.Cu") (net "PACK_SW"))
 (segment (start 118 112.7) (end 120 118) (width 1) (layer "B.Cu") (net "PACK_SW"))
 (segment (start 120 118) (end 149 118) (width 1) (layer "B.Cu") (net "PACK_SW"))
 (segment (start 149 118) (end 149 121.72) (width 1) (layer "B.Cu") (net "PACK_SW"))
 (segment (start 114 112.7) (end 111.636 126.08) (width 1.5) (layer "B.Cu") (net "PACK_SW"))
 (segment (start 111.636 126.08) (end 101.2 130) (width 1) (layer "B.Cu") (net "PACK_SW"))
 (segment (start 101.2 130) (end 101.2 141) (width 1) (layer "B.Cu") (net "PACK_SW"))
 (segment (start 101.2 141) (end 103 141) (width 1) (layer "B.Cu") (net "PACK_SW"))
 (segment (start 149 121.72) (end 154.9 121.72) (width 1) (layer "B.Cu") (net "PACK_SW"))
 (segment (start 106 128.62) (end 106 126.08) (width 0.8) (layer "B.Cu") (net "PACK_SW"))
 (segment (start 106 126.08) (end 111.636 126.08) (width 0.8) (layer "B.Cu") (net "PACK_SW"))
 (segment (start 123.7 155) (end 119 155) (width 0.5) (layer "F.Cu") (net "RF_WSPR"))
 (segment (start 119 155) (end 112 157) (width 0.5) (layer "F.Cu") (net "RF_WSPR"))
 (segment (start 112 157) (end 112 162) (width 0.5) (layer "F.Cu") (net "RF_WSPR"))
 (segment (start 159 118) (end 160.84 118) (width 0.3) (layer "B.Cu") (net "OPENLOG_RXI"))
 (segment (start 160.84 118) (end 160.84 112.8) (width 0.3) (layer "B.Cu") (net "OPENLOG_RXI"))
 (via (at 160.84 112.8) (size 0.8) (drill 0.4) (layers "F.Cu" "B.Cu") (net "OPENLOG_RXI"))
 (segment (start 160.84 112.8) (end 160.84 111.2) (width 0.3) (layer "F.Cu") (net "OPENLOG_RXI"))
 (via (at 160.84 111.2) (size 0.8) (drill 0.4) (layers "F.Cu" "B.Cu") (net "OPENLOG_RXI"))
 (segment (start 160.84 111.2) (end 160.84 110) (width 0.3) (layer "B.Cu") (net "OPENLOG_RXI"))
 (segment (start 103 108) (end 114 108) (width 1.5) (layer "F.Cu") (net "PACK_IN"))
 (segment (start 106 121) (end 100.8 121) (width 0.5) (layer "F.Cu") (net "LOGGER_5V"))
 (segment (start 100.8 121) (end 100.8 132) (width 0.5) (layer "F.Cu") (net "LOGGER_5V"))
 (segment (start 100.8 132) (end 107 132) (width 0.5) (layer "F.Cu") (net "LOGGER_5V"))
 (segment (start 107 132) (end 121.62 132) (width 0.5) (layer "F.Cu") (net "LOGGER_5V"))
 (segment (start 107.7 133.3) (end 107.7 132) (width 0.5) (layer "F.Cu") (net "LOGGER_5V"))
 (segment (start 103 115.5) (end 101.2 115.5) (width 0.5) (layer "F.Cu") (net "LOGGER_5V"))
 (segment (start 165.92 110) (end 165.92 112) (width 0.5) (layer "F.Cu") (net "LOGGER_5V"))
 (segment (start 165.92 112) (end 173 112) (width 0.5) (layer "F.Cu") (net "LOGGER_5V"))
 (segment (start 173 112) (end 173 121) (width 0.5) (layer "F.Cu") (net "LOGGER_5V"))
 (segment (start 110.24 133.3) (end 110.5 133.3) (width 0.4) (layer "F.Cu") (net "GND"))
 (segment (start 110.5 133.3) (end 110.5 140.62) (width 0.4) (layer "F.Cu") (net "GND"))
 (segment (start 108.08 115.5) (end 108 115.5) (width 0.4) (layer "B.Cu") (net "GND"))
 (segment (start 110.5 140.62) (end 114 140.62) (width 0.4) (layer "F.Cu") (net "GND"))
 (segment (start 112 140.62) (end 121.62 140.62) (width 0.6) (layer "F.Cu") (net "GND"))
 (segment (start 121.62 140.62) (end 120 140) (width 0.6) (layer "B.Cu") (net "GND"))
 (segment (start 121.62 140.62) (end 121.62 144) (width 0.4) (layer "B.Cu") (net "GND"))
 (segment (start 121.62 144) (end 120.78 149) (width 0.6) (layer "B.Cu") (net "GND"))
 (segment (start 161 121.5) (end 159.5 121.5) (width 0.4) (layer "B.Cu") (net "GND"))
 (segment (start 161 124.04) (end 159.5 124.04) (width 0.4) (layer "B.Cu") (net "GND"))
 (segment (start 161 126.58) (end 159.5 126.58) (width 0.4) (layer "B.Cu") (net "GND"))
 (segment (start 159.5 121.5) (end 159.5 139.28) (width 0.4) (layer "B.Cu") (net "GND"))
 (segment (start 159.5 139.28) (end 161 139.28) (width 0.4) (layer "B.Cu") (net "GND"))
 (segment (start 159.5 139.28) (end 159.5 141.5) (width 0.4) (layer "B.Cu") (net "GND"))
 (segment (start 159.5 141.5) (end 178 141.5) (width 0.4) (layer "B.Cu") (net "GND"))
 (segment (start 178.08 115) (end 178 115) (width 0.4) (layer "B.Cu") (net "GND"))
 (segment (start 175.54 121) (end 178 121) (width 0.4) (layer "B.Cu") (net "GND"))
 (segment (start 175.54 132) (end 178 132) (width 0.4) (layer "B.Cu") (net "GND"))
 (segment (start 154.9 131.912) (end 157 131.912) (width 0.4) (layer "F.Cu") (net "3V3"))
 (segment (start 157 131.912) (end 157 119.5) (width 0.4) (layer "F.Cu") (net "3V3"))
 (segment (start 157 119.5) (end 168.62 119.5) (width 0.4) (layer "F.Cu") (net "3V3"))
 (segment (start 168.62 119.5) (end 168.62 121.5) (width 0.4) (layer "F.Cu") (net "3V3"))
 (segment (start 168.62 121.5) (end 171 121.5) (width 0.4) (layer "F.Cu") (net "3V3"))
 (segment (start 171 121.5) (end 171 132) (width 0.4) (layer "F.Cu") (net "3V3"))
 (segment (start 171 132) (end 173 132) (width 0.4) (layer "F.Cu") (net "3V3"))
 (segment (start 173 132) (end 173 129) (width 0.4) (layer "F.Cu") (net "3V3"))
 (segment (start 173 129) (end 177 129) (width 0.4) (layer "F.Cu") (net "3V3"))
 (segment (start 177 129) (end 177 147) (width 0.4) (layer "F.Cu") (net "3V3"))
 (segment (start 177 147) (end 160 147) (width 0.4) (layer "F.Cu") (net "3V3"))
 (segment (start 160 147) (end 160 145) (width 0.4) (layer "F.Cu") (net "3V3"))
 (segment (start 154.9 137.008) (end 157 137.008) (width 0.3) (layer "B.Cu") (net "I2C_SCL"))
 (segment (start 157 137.008) (end 157 120) (width 0.3) (layer "B.Cu") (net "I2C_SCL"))
 (segment (start 157 120) (end 163 120) (width 0.3) (layer "B.Cu") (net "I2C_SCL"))
 (segment (start 163 120) (end 163 126.58) (width 0.3) (layer "B.Cu") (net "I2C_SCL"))
 (segment (start 163 126.58) (end 168.62 126.58) (width 0.3) (layer "B.Cu") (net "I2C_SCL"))
 (segment (start 154.9 139.556) (end 150 139.556) (width 0.3) (layer "F.Cu") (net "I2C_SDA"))
 (via (at 150 139.556) (size 0.8) (drill 0.4) (layers "F.Cu" "B.Cu") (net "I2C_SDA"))
 (segment (start 150 139.556) (end 150 123) (width 0.3) (layer "B.Cu") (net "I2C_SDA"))
 (segment (start 150 123) (end 147 123) (width 0.3) (layer "B.Cu") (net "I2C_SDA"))
 (via (at 147 123) (size 0.8) (drill 0.4) (layers "F.Cu" "B.Cu") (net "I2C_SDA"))
 (segment (start 147 123) (end 147 120.5) (width 0.3) (layer "F.Cu") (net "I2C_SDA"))
 (via (at 147 120.5) (size 0.8) (drill 0.4) (layers "F.Cu" "B.Cu") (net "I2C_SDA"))
 (segment (start 147 120.5) (end 147 119.2) (width 0.3) (layer "B.Cu") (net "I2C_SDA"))
 (via (at 147 119.2) (size 0.8) (drill 0.4) (layers "F.Cu" "B.Cu") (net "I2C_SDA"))
 (segment (start 147 119.2) (end 147 116.8) (width 0.3) (layer "F.Cu") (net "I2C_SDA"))
 (via (at 147 116.8) (size 0.8) (drill 0.4) (layers "F.Cu" "B.Cu") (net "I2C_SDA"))
 (segment (start 147 116.8) (end 147 112) (width 0.3) (layer "B.Cu") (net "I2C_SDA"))
 (segment (start 147 112) (end 164.5 112) (width 0.3) (layer "B.Cu") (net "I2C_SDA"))
 (segment (start 164.5 112) (end 164.5 124.04) (width 0.3) (layer "B.Cu") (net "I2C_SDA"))
 (segment (start 164.5 124.04) (end 168.62 124.04) (width 0.3) (layer "B.Cu") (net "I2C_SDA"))
 (segment (start 161 129.12) (end 158.5 129.12) (width 0.3) (layer "F.Cu") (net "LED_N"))
 (segment (start 158.5 129.12) (end 158.5 143) (width 0.3) (layer "F.Cu") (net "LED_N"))
 (segment (start 158.5 143) (end 173 143) (width 0.3) (layer "F.Cu") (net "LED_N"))
 (segment (start 173 143) (end 173 145) (width 0.3) (layer "F.Cu") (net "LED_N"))
 (segment (start 167.62 145) (end 170.46 145) (width 0.3) (layer "F.Cu") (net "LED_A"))
 (segment (start 154.9 126.816) (end 150.5 126.816) (width 0.3) (layer "F.Cu") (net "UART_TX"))
 (segment (start 150.5 126.816) (end 150.5 106) (width 0.3) (layer "F.Cu") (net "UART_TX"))
 (segment (start 150.5 106) (end 155.8 106) (width 0.3) (layer "F.Cu") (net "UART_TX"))
 (segment (start 155.8 106) (end 155.8 114) (width 0.3) (layer "F.Cu") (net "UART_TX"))
 (segment (start 155.8 114) (end 166.62 114) (width 0.3) (layer "F.Cu") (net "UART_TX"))
 (segment (start 166.62 114) (end 166.62 118) (width 0.3) (layer "F.Cu") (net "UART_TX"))
 (segment (start 154.9 129.364) (end 124 129.364) (width 0.3) (layer "F.Cu") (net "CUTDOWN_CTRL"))
 (segment (start 124 129.364) (end 124 134.5) (width 0.3) (layer "F.Cu") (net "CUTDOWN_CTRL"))
 (segment (start 124 134.5) (end 124 136.8) (width 0.3) (layer "F.Cu") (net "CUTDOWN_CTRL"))
 (segment (start 124 136.8) (end 115.5 136.8) (width 0.3) (layer "F.Cu") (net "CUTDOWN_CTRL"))
 (segment (start 115.5 136.8) (end 114 135.54) (width 0.3) (layer "F.Cu") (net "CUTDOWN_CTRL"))
 (segment (start 121.62 135.54) (end 121.62 138.08) (width 0.3) (layer "B.Cu") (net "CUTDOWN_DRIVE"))
 (segment (start 121.62 138.08) (end 123 138.08) (width 0.3) (layer "B.Cu") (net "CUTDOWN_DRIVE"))
 (segment (start 123 138.08) (end 124.5 138.08) (width 0.3) (layer "B.Cu") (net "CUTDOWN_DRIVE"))
 (segment (start 124.5 138.08) (end 124.5 130) (width 0.3) (layer "B.Cu") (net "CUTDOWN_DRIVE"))
 (segment (start 124.5 130) (end 111.5 130) (width 0.3) (layer "B.Cu") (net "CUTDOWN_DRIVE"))
 (segment (start 111.5 130) (end 111.5 146) (width 0.3) (layer "B.Cu") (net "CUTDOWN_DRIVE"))
 (segment (start 111.5 146) (end 103 146) (width 0.3) (layer "B.Cu") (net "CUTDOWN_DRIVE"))
 (segment (start 103 146) (end 103 148) (width 0.3) (layer "B.Cu") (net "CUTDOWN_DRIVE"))
 (segment (start 110.62 148) (end 114 148) (width 0.3) (layer "B.Cu") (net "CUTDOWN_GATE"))
 (segment (start 114 144) (end 114 148) (width 0.3) (layer "B.Cu") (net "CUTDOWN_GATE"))
 (segment (start 114 148) (end 115.7 149) (width 0.3) (layer "B.Cu") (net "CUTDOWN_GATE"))
 (segment (start 103 138.5) (end 105 138.5) (width 1.5) (layer "F.Cu") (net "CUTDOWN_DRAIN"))
 (segment (start 105 138.5) (end 105 143) (width 1.5) (layer "F.Cu") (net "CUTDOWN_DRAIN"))
 (segment (start 105 143) (end 108 146) (width 1.5) (layer "F.Cu") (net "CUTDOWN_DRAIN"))
 (segment (start 108 146) (end 118.24 146) (width 1.5) (layer "F.Cu") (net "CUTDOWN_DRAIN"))
 (segment (start 118.24 146) (end 118.24 149) (width 1.5) (layer "F.Cu") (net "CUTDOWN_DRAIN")))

